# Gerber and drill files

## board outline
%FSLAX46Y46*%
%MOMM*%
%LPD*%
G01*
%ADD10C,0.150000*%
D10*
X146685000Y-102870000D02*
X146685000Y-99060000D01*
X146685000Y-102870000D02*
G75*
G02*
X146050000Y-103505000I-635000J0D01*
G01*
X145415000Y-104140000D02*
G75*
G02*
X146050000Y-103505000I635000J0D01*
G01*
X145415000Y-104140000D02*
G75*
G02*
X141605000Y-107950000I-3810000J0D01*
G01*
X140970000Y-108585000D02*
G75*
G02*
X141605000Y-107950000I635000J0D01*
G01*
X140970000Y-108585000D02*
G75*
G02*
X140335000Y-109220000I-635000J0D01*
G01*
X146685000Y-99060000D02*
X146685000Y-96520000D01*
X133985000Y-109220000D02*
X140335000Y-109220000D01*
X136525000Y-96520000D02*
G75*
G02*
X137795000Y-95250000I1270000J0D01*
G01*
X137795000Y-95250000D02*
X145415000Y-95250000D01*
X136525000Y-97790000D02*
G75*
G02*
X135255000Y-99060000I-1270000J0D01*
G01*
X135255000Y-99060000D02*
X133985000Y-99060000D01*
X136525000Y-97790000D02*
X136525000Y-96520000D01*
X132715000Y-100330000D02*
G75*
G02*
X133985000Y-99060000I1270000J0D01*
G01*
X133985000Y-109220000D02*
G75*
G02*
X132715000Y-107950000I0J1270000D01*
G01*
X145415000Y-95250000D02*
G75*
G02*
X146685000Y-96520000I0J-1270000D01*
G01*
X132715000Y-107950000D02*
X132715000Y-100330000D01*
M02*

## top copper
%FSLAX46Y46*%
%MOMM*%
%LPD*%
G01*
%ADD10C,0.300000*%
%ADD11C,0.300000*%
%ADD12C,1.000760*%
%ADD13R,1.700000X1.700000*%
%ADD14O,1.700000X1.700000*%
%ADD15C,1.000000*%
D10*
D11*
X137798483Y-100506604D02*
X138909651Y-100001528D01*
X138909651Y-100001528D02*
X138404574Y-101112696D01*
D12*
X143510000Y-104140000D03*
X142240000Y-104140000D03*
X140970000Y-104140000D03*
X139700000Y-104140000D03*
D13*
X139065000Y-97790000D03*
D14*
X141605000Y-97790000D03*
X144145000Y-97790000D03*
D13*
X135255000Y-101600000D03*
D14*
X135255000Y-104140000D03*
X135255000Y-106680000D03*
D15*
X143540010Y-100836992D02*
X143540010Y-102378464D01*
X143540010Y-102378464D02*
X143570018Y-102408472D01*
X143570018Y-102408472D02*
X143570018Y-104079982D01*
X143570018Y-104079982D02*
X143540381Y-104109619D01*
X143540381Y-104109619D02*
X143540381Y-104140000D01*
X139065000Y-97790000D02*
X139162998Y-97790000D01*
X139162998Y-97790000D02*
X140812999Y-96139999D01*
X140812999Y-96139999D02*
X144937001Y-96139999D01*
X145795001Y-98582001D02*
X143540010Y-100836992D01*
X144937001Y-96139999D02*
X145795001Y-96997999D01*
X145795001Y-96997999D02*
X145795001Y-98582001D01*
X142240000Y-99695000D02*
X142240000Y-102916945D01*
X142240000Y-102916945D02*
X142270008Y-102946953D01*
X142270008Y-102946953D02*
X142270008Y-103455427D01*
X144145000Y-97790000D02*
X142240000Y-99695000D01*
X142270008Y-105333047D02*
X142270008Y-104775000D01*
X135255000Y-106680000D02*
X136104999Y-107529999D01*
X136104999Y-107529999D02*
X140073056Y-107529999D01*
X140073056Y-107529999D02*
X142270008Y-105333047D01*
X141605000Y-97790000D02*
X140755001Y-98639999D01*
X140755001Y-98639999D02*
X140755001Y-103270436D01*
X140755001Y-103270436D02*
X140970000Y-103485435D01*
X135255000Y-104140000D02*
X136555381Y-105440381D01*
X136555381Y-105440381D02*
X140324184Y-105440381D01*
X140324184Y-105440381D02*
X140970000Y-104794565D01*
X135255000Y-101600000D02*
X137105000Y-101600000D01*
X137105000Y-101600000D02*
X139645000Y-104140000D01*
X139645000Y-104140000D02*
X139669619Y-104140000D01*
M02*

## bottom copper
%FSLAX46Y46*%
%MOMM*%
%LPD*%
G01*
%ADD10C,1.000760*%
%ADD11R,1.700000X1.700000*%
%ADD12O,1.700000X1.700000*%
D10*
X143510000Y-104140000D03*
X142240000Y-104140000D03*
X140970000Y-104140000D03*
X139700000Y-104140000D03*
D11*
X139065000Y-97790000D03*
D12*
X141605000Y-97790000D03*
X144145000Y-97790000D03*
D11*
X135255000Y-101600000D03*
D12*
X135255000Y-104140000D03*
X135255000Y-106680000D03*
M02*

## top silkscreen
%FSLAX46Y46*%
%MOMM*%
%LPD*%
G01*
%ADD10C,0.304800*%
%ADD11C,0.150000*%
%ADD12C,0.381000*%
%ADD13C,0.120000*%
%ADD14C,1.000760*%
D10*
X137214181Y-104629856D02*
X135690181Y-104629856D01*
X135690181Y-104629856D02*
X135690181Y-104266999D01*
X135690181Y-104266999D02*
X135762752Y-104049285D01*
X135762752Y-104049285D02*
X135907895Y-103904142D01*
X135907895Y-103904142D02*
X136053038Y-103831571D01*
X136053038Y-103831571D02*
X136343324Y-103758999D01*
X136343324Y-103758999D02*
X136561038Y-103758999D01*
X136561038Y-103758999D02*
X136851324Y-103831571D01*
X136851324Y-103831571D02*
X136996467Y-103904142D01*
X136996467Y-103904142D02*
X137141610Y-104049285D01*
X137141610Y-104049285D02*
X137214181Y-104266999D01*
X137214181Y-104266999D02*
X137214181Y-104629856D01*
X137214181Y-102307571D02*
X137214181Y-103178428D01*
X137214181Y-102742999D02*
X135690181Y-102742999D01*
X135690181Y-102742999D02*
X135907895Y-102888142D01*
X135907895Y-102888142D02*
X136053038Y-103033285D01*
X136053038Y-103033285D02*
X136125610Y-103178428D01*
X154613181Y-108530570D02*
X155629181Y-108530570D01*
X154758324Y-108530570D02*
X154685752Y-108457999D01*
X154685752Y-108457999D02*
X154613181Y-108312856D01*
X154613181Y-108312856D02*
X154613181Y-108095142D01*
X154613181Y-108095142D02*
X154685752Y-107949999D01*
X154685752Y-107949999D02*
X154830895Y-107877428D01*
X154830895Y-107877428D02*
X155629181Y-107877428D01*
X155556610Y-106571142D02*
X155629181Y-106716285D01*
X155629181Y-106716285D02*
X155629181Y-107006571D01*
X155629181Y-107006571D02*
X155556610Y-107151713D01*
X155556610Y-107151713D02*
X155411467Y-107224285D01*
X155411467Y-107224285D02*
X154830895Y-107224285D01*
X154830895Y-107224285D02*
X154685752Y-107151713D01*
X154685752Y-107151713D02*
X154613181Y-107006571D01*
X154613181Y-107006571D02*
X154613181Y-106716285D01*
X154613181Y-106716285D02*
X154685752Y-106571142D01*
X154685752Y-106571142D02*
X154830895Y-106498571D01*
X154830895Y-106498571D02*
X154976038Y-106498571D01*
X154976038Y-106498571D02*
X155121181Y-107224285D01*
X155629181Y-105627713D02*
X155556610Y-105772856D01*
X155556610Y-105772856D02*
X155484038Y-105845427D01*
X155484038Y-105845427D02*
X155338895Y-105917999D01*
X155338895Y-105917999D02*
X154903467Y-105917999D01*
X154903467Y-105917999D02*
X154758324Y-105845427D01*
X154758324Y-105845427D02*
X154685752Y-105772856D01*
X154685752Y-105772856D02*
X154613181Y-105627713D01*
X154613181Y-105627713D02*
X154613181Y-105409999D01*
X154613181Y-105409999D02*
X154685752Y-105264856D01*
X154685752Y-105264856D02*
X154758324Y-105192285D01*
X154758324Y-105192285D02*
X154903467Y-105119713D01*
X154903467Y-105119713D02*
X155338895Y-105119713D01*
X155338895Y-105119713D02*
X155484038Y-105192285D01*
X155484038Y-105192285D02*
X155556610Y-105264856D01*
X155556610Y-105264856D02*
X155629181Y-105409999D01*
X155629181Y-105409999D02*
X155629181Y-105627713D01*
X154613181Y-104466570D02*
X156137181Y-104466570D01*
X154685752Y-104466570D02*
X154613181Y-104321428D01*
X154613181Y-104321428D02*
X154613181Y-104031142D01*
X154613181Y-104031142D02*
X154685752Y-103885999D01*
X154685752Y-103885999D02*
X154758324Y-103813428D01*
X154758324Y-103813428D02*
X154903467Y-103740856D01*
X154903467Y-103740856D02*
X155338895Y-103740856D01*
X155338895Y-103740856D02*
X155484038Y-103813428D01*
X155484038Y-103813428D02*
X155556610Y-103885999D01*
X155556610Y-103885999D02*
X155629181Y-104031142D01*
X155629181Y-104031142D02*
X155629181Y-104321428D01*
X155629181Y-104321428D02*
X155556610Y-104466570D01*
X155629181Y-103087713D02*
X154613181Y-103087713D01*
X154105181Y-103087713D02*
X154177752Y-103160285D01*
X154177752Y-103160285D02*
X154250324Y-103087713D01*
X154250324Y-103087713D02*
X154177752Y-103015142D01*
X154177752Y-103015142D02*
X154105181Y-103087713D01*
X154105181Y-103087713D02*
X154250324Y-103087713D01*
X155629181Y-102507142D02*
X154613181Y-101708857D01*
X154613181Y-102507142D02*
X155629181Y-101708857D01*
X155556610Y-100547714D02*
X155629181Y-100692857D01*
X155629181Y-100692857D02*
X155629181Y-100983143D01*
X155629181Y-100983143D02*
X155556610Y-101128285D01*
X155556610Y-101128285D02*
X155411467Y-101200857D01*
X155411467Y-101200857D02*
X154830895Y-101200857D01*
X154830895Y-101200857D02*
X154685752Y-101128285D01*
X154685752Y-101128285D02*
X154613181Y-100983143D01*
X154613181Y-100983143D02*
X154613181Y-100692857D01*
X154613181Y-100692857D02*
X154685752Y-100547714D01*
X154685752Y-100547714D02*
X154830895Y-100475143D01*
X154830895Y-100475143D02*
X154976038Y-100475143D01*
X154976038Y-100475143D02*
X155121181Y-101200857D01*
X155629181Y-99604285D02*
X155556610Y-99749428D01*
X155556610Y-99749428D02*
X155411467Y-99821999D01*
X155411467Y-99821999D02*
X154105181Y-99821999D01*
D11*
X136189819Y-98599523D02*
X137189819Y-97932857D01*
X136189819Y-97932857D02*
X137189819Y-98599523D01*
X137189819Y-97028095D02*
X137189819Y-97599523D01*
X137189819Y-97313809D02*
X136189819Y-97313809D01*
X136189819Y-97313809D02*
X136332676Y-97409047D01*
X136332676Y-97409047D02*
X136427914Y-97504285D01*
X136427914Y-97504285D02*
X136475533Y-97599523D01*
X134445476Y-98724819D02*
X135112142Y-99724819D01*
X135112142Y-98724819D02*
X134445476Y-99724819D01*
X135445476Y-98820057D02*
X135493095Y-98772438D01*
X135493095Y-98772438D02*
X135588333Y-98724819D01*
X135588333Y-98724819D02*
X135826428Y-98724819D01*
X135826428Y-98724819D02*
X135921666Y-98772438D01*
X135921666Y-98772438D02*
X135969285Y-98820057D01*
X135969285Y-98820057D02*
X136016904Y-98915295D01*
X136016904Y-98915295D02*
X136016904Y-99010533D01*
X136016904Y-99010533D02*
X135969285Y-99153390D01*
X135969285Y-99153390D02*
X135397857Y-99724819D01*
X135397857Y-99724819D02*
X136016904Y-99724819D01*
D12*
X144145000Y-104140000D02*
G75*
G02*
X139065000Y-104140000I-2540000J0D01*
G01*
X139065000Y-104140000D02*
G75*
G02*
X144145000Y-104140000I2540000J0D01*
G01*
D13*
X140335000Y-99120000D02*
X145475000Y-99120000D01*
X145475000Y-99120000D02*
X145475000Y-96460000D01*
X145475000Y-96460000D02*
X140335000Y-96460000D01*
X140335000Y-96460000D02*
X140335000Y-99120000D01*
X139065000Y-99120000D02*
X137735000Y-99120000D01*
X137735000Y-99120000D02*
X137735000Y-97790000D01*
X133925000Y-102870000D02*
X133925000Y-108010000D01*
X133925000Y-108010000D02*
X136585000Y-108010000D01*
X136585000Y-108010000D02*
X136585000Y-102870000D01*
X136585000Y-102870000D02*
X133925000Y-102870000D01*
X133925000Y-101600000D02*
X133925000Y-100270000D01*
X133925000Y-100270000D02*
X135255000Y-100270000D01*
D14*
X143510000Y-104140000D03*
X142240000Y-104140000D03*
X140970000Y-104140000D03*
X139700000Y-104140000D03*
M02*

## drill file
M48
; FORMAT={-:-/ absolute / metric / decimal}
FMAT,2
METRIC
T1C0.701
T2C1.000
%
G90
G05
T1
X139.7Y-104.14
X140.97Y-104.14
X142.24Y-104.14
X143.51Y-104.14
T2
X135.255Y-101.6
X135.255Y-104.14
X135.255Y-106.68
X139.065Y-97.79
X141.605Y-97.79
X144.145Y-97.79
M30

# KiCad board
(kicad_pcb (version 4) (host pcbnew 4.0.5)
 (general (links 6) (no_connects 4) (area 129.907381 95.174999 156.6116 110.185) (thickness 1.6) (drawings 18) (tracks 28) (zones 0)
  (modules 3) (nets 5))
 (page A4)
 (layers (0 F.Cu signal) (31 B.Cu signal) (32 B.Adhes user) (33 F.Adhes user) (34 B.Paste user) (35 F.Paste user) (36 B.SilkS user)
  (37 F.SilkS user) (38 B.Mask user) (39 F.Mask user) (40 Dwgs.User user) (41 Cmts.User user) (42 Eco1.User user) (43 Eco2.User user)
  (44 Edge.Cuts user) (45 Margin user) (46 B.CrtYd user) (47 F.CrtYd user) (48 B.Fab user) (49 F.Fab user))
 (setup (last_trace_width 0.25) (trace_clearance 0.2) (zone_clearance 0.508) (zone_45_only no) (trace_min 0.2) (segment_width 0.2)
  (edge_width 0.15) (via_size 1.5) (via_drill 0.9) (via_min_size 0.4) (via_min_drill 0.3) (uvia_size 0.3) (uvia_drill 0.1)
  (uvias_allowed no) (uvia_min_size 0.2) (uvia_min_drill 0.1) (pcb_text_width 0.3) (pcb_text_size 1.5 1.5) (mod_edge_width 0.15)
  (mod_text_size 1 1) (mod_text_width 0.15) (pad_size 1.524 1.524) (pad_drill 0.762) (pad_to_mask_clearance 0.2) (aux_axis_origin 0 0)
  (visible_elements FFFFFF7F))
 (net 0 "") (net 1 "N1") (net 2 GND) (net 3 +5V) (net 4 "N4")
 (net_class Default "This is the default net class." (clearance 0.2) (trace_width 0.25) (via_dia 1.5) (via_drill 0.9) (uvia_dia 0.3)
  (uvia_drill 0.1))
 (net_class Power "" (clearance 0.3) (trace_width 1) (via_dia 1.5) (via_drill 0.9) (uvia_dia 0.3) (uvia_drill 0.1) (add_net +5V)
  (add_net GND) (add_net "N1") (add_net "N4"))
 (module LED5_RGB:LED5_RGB (layer F.Cu) (at 141.605 104.14 180)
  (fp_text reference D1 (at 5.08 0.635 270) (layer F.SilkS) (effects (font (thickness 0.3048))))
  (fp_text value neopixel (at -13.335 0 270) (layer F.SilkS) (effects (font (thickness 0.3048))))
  (fp_circle (center 0 0) (end 2.54 0) (layer F.SilkS) (width 0.381))
  (pad 1 thru_hole circle (at -1.905 0 180) (size 1.00076 1.00076) (drill 0.70104) (layers *.Cu *.Mask F.SilkS) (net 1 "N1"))
  (pad 2 thru_hole circle (at -0.635 0 180) (size 1.00076 1.00076) (drill 0.70104) (layers *.Cu *.Mask F.SilkS) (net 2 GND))
  (pad 3 thru_hole circle (at 0.635 0 180) (size 1.00076 1.00076) (drill 0.70104) (layers *.Cu *.Mask F.SilkS) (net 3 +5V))
  (pad 4 thru_hole circle (at 1.905 0 180) (size 1.00076 1.00076) (drill 0.70104) (layers *.Cu *.Mask F.SilkS) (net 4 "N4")))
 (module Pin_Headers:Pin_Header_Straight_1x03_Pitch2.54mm (layer F.Cu) (at 139.065 97.79 90)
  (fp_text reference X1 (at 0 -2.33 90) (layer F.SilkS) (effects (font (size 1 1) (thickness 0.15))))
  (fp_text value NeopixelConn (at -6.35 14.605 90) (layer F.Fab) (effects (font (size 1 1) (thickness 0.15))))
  (fp_line (start -1.33 1.27) (end -1.33 6.41) (layer F.SilkS) (width 0.12))
  (fp_line (start -1.33 6.41) (end 1.33 6.41) (layer F.SilkS) (width 0.12))
  (fp_line (start 1.33 6.41) (end 1.33 1.27) (layer F.SilkS) (width 0.12))
  (fp_line (start 1.33 1.27) (end -1.33 1.27) (layer F.SilkS) (width 0.12))
  (fp_line (start -1.33 0) (end -1.33 -1.33) (layer F.SilkS) (width 0.12))
  (fp_line (start -1.33 -1.33) (end 0 -1.33) (layer F.SilkS) (width 0.12))
  (pad 1 thru_hole rect (at 0 0 90) (size 1.7 1.7) (drill 1) (layers *.Cu *.Mask) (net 1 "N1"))
  (pad 2 thru_hole oval (at 0 2.54 90) (size 1.7 1.7) (drill 1) (layers *.Cu *.Mask) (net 3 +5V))
  (pad 3 thru_hole oval (at 0 5.08 90) (size 1.7 1.7) (drill 1) (layers *.Cu *.Mask) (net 2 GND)))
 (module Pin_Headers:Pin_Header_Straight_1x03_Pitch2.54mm (layer F.Cu) (at 135.255 101.6)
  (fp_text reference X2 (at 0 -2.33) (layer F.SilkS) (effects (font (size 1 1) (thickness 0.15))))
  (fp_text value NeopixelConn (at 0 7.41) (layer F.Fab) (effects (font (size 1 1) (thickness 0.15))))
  (fp_line (start -1.33 1.27) (end -1.33 6.41) (layer F.SilkS) (width 0.12))
  (fp_line (start -1.33 6.41) (end 1.33 6.41) (layer F.SilkS) (width 0.12))
  (fp_line (start 1.33 6.41) (end 1.33 1.27) (layer F.SilkS) (width 0.12))
  (fp_line (start 1.33 1.27) (end -1.33 1.27) (layer F.SilkS) (width 0.12))
  (fp_line (start -1.33 0) (end -1.33 -1.33) (layer F.SilkS) (width 0.12))
  (fp_line (start -1.33 -1.33) (end 0 -1.33) (layer F.SilkS) (width 0.12))
  (pad 1 thru_hole rect (at 0 0) (size 1.7 1.7) (drill 1) (layers *.Cu *.Mask) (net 4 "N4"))
  (pad 2 thru_hole oval (at 0 2.54) (size 1.7 1.7) (drill 1) (layers *.Cu *.Mask) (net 3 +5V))
  (pad 3 thru_hole oval (at 0 5.08) (size 1.7 1.7) (drill 1) (layers *.Cu *.Mask) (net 2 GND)))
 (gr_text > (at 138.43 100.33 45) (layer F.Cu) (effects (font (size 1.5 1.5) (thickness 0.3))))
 (gr_line (start 146.685 102.87) (end 146.685 99.06) (layer Edge.Cuts) (width 0.15))
 (gr_arc (start 146.05 102.87) (end 146.685 102.87) (angle 90) (layer Edge.Cuts) (width 0.15))
 (gr_arc (start 146.05 104.14) (end 145.415 104.14) (angle 90) (layer Edge.Cuts) (width 0.15))
 (gr_arc (start 141.605 104.14) (end 145.415 104.14) (angle 90) (layer Edge.Cuts) (width 0.15))
 (gr_arc (start 141.605 108.585) (end 140.97 108.585) (angle 90) (layer Edge.Cuts) (width 0.15))
 (gr_arc (start 140.335 108.585) (end 140.97 108.585) (angle 90) (layer Edge.Cuts) (width 0.15))
 (gr_line (start 146.685 99.06) (end 146.685 96.52) (layer Edge.Cuts) (width 0.15))
 (gr_line (start 133.985 109.22) (end 140.335 109.22) (layer Edge.Cuts) (width 0.15))
 (gr_arc (start 137.795 96.52) (end 136.525 96.52) (angle 90) (layer Edge.Cuts) (width 0.15))
 (gr_line (start 137.795 95.25) (end 145.415 95.25) (layer Edge.Cuts) (width 0.15))
 (gr_arc (start 135.255 97.79) (end 136.525 97.79) (angle 90) (layer Edge.Cuts) (width 0.15))
 (gr_line (start 135.255 99.06) (end 133.985 99.06) (layer Edge.Cuts) (width 0.15))
 (gr_line (start 136.525 97.79) (end 136.525 96.52) (layer Edge.Cuts) (width 0.15))
 (gr_arc (start 133.985 100.33) (end 132.715 100.33) (angle 90) (layer Edge.Cuts) (width 0.15))
 (gr_arc (start 133.985 107.95) (end 133.985 109.22) (angle 90) (layer Edge.Cuts) (width 0.15))
 (gr_arc (start 145.415 96.52) (end 145.415 95.25) (angle 90) (layer Edge.Cuts) (width 0.15))
 (gr_line (start 132.715 107.95) (end 132.715 100.33) (layer Edge.Cuts) (width 0.15))
 (segment (start 143.54001 100.836992) (end 143.54001 102.378464) (width 1) (layer F.Cu) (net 1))
 (segment (start 143.54001 102.378464) (end 143.570018 102.408472) (width 1) (layer F.Cu) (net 1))
 (segment (start 143.570018 102.408472) (end 143.570018 104.079982) (width 1) (layer F.Cu) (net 1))
 (segment (start 143.570018 104.079982) (end 143.540381 104.109619) (width 1) (layer F.Cu) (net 1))
 (segment (start 143.540381 104.109619) (end 143.540381 104.14) (width 1) (layer F.Cu) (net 1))
 (segment (start 139.065 97.79) (end 139.162998 97.79) (width 1) (layer F.Cu) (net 1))
 (segment (start 139.162998 97.79) (end 140.812999 96.139999) (width 1) (layer F.Cu) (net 1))
 (segment (start 140.812999 96.139999) (end 144.937001 96.139999) (width 1) (layer F.Cu) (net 1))
 (segment (start 145.795001 98.582001) (end 143.54001 100.836992) (width 1) (layer F.Cu) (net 1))
 (segment (start 144.937001 96.139999) (end 145.795001 96.997999) (width 1) (layer F.Cu) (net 1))
 (segment (start 145.795001 96.997999) (end 145.795001 98.582001) (width 1) (layer F.Cu) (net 1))
 (segment (start 142.24 99.695) (end 142.24 102.916945) (width 1) (layer F.Cu) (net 2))
 (segment (start 142.24 102.916945) (end 142.270008 102.946953) (width 1) (layer F.Cu) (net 2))
 (segment (start 142.270008 102.946953) (end 142.270008 103.455427) (width 1) (layer F.Cu) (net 2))
 (segment (start 144.145 97.79) (end 142.24 99.695) (width 1) (layer F.Cu) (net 2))
 (segment (start 142.270008 105.333047) (end 142.270008 104.775) (width 1) (layer F.Cu) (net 2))
 (segment (start 135.255 106.68) (end 136.104999 107.529999) (width 1) (layer F.Cu) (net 2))
 (segment (start 136.104999 107.529999) (end 140.073056 107.529999) (width 1) (layer F.Cu) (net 2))
 (segment (start 140.073056 107.529999) (end 142.270008 105.333047) (width 1) (layer F.Cu) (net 2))
 (segment (start 141.605 97.79) (end 140.755001 98.639999) (width 1) (layer F.Cu) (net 3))
 (segment (start 140.755001 98.639999) (end 140.755001 103.270436) (width 1) (layer F.Cu) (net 3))
 (segment (start 140.755001 103.270436) (end 140.97 103.485435) (width 1) (layer F.Cu) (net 3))
 (segment (start 135.255 104.14) (end 136.555381 105.440381) (width 1) (layer F.Cu) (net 3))
 (segment (start 136.555381 105.440381) (end 140.324184 105.440381) (width 1) (layer F.Cu) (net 3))
 (segment (start 140.324184 105.440381) (end 140.97 104.794565) (width 1) (layer F.Cu) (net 3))
 (segment (start 135.255 101.6) (end 137.105 101.6) (width 1) (layer F.Cu) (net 4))
 (segment (start 137.105 101.6) (end 139.645 104.14) (width 1) (layer F.Cu) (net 4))
 (segment (start 139.645 104.14) (end 139.669619 104.14) (width 1) (layer F.Cu) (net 4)))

